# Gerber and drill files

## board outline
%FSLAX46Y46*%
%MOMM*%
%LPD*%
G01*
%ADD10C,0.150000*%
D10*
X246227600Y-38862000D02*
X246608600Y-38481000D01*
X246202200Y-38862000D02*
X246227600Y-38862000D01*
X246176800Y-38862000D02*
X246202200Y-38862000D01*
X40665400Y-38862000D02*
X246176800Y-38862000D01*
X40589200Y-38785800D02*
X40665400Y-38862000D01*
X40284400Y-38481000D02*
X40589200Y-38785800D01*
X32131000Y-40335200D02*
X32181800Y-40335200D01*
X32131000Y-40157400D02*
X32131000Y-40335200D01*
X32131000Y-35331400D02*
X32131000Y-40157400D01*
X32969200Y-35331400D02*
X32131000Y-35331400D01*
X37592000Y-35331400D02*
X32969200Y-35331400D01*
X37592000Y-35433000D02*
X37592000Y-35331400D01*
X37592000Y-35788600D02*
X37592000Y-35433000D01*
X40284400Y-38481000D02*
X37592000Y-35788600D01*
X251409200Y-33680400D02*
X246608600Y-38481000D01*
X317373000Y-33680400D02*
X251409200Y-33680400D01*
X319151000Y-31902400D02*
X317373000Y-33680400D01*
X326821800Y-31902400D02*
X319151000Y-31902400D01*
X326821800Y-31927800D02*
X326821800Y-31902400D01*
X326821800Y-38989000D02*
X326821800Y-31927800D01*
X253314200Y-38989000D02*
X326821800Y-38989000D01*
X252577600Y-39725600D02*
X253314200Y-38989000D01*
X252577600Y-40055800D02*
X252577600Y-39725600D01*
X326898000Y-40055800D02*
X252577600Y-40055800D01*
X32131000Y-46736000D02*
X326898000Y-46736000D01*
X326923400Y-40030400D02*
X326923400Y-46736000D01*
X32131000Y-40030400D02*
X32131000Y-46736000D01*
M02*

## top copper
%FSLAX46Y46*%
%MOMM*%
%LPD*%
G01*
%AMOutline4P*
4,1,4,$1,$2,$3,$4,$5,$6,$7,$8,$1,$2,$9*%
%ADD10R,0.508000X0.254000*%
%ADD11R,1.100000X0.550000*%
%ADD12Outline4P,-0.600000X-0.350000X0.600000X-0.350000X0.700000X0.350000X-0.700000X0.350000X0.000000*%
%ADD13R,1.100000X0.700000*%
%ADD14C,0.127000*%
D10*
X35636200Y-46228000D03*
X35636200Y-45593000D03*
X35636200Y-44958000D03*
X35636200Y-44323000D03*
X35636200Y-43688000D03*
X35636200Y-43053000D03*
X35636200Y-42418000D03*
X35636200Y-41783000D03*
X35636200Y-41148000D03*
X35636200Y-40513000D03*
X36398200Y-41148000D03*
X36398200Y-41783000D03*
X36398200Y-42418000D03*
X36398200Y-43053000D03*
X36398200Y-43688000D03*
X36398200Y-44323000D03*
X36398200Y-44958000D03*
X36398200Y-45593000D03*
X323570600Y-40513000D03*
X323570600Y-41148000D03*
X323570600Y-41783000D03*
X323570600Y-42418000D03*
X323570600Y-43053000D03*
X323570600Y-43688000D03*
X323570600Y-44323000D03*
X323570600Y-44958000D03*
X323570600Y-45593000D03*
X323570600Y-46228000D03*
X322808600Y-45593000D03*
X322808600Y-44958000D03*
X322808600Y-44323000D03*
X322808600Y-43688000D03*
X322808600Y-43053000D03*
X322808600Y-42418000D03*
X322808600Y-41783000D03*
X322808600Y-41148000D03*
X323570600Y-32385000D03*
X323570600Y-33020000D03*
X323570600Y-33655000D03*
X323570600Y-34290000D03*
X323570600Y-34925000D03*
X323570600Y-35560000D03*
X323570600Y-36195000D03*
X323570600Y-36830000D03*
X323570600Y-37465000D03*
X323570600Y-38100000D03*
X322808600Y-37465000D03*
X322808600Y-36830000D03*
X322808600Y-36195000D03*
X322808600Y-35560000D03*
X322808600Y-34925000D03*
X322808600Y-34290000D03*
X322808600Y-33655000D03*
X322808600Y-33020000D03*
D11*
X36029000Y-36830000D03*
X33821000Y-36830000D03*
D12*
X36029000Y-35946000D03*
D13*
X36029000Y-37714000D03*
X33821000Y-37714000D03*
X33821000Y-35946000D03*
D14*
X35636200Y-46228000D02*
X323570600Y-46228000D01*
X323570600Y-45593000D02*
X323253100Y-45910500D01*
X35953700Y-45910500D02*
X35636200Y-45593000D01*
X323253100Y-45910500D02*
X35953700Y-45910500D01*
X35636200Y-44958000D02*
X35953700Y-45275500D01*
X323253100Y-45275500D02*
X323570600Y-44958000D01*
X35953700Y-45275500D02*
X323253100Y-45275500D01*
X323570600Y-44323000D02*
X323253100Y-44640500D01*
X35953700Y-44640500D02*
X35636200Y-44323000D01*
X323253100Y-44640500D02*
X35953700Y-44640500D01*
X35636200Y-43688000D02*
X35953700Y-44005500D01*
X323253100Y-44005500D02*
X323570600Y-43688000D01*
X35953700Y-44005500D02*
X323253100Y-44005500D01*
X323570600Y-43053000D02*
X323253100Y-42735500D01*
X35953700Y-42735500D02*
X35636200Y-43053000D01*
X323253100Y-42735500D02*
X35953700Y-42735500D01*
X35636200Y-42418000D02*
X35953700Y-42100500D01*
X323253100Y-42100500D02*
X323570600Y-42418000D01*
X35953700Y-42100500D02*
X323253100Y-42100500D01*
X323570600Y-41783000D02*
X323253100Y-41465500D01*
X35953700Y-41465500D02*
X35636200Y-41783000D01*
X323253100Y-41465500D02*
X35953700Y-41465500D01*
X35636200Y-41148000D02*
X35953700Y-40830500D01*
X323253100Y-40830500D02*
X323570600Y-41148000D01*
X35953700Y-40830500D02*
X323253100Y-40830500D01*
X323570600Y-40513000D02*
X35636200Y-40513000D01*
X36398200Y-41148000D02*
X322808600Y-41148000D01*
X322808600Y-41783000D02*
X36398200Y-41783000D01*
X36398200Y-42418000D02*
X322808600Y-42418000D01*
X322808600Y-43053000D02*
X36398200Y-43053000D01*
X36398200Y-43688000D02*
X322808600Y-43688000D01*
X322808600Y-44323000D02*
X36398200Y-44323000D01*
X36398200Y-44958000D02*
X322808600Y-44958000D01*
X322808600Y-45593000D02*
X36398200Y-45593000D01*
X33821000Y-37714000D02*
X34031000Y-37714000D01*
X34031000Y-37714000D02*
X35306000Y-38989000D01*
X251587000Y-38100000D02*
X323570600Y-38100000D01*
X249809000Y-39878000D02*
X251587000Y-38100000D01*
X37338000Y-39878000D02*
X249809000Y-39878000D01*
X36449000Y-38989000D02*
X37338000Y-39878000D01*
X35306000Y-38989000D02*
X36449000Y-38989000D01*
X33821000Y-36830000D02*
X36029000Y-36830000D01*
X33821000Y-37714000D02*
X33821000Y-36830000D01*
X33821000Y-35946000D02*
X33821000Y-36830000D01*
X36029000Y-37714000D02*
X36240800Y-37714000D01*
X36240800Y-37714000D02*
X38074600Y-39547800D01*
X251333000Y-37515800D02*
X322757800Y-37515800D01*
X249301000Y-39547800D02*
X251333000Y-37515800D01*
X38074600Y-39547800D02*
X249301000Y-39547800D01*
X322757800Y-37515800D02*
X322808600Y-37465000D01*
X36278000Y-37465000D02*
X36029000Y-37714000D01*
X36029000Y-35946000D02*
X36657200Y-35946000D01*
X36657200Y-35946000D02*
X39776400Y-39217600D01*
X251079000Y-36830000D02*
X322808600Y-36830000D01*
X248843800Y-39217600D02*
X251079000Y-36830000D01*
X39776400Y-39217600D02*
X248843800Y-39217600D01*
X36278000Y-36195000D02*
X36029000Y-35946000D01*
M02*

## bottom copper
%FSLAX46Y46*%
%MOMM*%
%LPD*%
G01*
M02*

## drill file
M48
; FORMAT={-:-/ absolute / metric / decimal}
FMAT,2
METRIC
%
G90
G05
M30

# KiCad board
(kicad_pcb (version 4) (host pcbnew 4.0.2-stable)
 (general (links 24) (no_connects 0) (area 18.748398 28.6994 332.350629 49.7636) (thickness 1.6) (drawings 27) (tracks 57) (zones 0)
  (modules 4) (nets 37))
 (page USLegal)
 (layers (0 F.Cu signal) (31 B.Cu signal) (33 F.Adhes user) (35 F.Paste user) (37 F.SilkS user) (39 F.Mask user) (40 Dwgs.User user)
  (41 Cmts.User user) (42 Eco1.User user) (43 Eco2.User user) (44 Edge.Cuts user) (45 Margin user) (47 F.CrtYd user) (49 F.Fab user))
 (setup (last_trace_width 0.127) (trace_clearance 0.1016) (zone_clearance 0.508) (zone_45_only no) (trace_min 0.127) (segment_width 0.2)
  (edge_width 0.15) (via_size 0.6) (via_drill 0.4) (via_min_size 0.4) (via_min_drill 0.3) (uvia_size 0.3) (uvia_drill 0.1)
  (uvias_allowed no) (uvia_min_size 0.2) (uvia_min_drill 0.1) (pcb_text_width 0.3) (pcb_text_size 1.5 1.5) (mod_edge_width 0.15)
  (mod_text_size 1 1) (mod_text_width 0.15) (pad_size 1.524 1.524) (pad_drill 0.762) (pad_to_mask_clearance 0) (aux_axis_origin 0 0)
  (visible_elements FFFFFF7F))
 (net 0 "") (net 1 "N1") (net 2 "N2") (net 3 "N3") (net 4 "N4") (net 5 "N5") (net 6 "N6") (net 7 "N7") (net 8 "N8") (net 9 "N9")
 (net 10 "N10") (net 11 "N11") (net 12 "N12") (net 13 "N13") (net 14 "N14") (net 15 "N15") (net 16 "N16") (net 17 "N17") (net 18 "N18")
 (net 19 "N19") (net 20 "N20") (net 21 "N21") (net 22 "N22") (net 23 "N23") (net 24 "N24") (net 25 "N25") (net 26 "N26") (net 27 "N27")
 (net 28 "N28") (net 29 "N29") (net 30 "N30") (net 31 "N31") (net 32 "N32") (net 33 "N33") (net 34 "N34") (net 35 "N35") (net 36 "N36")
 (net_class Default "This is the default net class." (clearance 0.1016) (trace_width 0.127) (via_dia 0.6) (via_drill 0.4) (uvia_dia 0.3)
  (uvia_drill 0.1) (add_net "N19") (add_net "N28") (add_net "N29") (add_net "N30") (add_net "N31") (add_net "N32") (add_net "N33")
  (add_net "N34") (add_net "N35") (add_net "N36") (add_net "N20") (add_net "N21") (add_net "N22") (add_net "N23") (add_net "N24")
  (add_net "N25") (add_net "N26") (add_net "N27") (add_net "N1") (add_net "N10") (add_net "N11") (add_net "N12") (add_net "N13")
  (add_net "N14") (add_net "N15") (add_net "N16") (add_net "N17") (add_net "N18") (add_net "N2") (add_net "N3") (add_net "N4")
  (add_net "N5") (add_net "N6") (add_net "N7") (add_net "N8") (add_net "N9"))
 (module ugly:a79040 (layer F.Cu) (at 33.4772 43.307)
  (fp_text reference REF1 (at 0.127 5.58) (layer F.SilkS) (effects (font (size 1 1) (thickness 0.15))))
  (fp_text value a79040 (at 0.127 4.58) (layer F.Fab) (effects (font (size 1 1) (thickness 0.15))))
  (pad 1 smd rect (at 2.159 2.921) (size 0.508 0.254) (layers F.Cu F.Paste F.Mask) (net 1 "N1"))
  (pad 2 smd rect (at 2.159 2.286) (size 0.508 0.254) (layers F.Cu F.Paste F.Mask) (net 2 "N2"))
  (pad 3 smd rect (at 2.159 1.651) (size 0.508 0.254) (layers F.Cu F.Paste F.Mask) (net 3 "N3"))
  (pad 4 smd rect (at 2.159 1.016) (size 0.508 0.254) (layers F.Cu F.Paste F.Mask) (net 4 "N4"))
  (pad 5 smd rect (at 2.159 0.381) (size 0.508 0.254) (layers F.Cu F.Paste F.Mask) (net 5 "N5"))
  (pad 6 smd rect (at 2.159 -0.254) (size 0.508 0.254) (layers F.Cu F.Paste F.Mask) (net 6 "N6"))
  (pad 7 smd rect (at 2.159 -0.889) (size 0.508 0.254) (layers F.Cu F.Paste F.Mask) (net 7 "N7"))
  (pad 8 smd rect (at 2.159 -1.524) (size 0.508 0.254) (layers F.Cu F.Paste F.Mask) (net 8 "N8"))
  (pad 9 smd rect (at 2.159 -2.159) (size 0.508 0.254) (layers F.Cu F.Paste F.Mask) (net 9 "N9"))
  (pad 10 smd rect (at 2.159 -2.794) (size 0.508 0.254) (layers F.Cu F.Paste F.Mask) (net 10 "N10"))
  (pad 11 smd rect (at 2.921 -2.159) (size 0.508 0.254) (layers F.Cu F.Paste F.Mask) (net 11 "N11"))
  (pad 12 smd rect (at 2.921 -1.524) (size 0.508 0.254) (layers F.Cu F.Paste F.Mask) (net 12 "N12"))
  (pad 13 smd rect (at 2.921 -0.889) (size 0.508 0.254) (layers F.Cu F.Paste F.Mask) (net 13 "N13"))
  (pad 14 smd rect (at 2.921 -0.254) (size 0.508 0.254) (layers F.Cu F.Paste F.Mask) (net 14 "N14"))
  (pad 15 smd rect (at 2.921 0.381) (size 0.508 0.254) (layers F.Cu F.Paste F.Mask) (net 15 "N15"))
  (pad 16 smd rect (at 2.921 1.016) (size 0.508 0.254) (layers F.Cu F.Paste F.Mask) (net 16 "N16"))
  (pad 17 smd rect (at 2.921 1.651) (size 0.508 0.254) (layers F.Cu F.Paste F.Mask) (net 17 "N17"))
  (pad 18 smd rect (at 2.921 2.286) (size 0.508 0.254) (layers F.Cu F.Paste F.Mask) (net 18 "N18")))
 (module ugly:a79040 (layer F.Cu) (at 325.7296 43.434 180)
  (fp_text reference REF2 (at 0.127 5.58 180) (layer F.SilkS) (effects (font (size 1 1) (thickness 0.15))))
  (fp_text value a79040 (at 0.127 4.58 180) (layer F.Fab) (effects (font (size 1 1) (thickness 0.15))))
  (pad 1 smd rect (at 2.159 2.921 180) (size 0.508 0.254) (layers F.Cu F.Paste F.Mask) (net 10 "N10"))
  (pad 2 smd rect (at 2.159 2.286 180) (size 0.508 0.254) (layers F.Cu F.Paste F.Mask) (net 9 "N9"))
  (pad 3 smd rect (at 2.159 1.651 180) (size 0.508 0.254) (layers F.Cu F.Paste F.Mask) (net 8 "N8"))
  (pad 4 smd rect (at 2.159 1.016 180) (size 0.508 0.254) (layers F.Cu F.Paste F.Mask) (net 7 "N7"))
  (pad 5 smd rect (at 2.159 0.381 180) (size 0.508 0.254) (layers F.Cu F.Paste F.Mask) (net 6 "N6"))
  (pad 6 smd rect (at 2.159 -0.254 180) (size 0.508 0.254) (layers F.Cu F.Paste F.Mask) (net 5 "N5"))
  (pad 7 smd rect (at 2.159 -0.889 180) (size 0.508 0.254) (layers F.Cu F.Paste F.Mask) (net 4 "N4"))
  (pad 8 smd rect (at 2.159 -1.524 180) (size 0.508 0.254) (layers F.Cu F.Paste F.Mask) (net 3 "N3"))
  (pad 9 smd rect (at 2.159 -2.159 180) (size 0.508 0.254) (layers F.Cu F.Paste F.Mask) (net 2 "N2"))
  (pad 10 smd rect (at 2.159 -2.794 180) (size 0.508 0.254) (layers F.Cu F.Paste F.Mask) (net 1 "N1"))
  (pad 11 smd rect (at 2.921 -2.159 180) (size 0.508 0.254) (layers F.Cu F.Paste F.Mask) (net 18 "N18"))
  (pad 12 smd rect (at 2.921 -1.524 180) (size 0.508 0.254) (layers F.Cu F.Paste F.Mask) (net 17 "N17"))
  (pad 13 smd rect (at 2.921 -0.889 180) (size 0.508 0.254) (layers F.Cu F.Paste F.Mask) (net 16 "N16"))
  (pad 14 smd rect (at 2.921 -0.254 180) (size 0.508 0.254) (layers F.Cu F.Paste F.Mask) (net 15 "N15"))
  (pad 15 smd rect (at 2.921 0.381 180) (size 0.508 0.254) (layers F.Cu F.Paste F.Mask) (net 14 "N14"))
  (pad 16 smd rect (at 2.921 1.016 180) (size 0.508 0.254) (layers F.Cu F.Paste F.Mask) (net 13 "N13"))
  (pad 17 smd rect (at 2.921 1.651 180) (size 0.508 0.254) (layers F.Cu F.Paste F.Mask) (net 12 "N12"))
  (pad 18 smd rect (at 2.921 2.286 180) (size 0.508 0.254) (layers F.Cu F.Paste F.Mask) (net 11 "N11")))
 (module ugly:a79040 (layer F.Cu) (at 325.7296 35.306 180)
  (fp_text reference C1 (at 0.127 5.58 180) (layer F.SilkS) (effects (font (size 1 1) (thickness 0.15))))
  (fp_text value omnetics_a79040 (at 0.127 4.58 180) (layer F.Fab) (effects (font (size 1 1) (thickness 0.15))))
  (pad 1 smd rect (at 2.159 2.921 180) (size 0.508 0.254) (layers F.Cu F.Paste F.Mask) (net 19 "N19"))
  (pad 2 smd rect (at 2.159 2.286 180) (size 0.508 0.254) (layers F.Cu F.Paste F.Mask) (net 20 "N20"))
  (pad 3 smd rect (at 2.159 1.651 180) (size 0.508 0.254) (layers F.Cu F.Paste F.Mask) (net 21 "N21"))
  (pad 4 smd rect (at 2.159 1.016 180) (size 0.508 0.254) (layers F.Cu F.Paste F.Mask) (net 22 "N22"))
  (pad 5 smd rect (at 2.159 0.381 180) (size 0.508 0.254) (layers F.Cu F.Paste F.Mask) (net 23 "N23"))
  (pad 6 smd rect (at 2.159 -0.254 180) (size 0.508 0.254) (layers F.Cu F.Paste F.Mask) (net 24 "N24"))
  (pad 7 smd rect (at 2.159 -0.889 180) (size 0.508 0.254) (layers F.Cu F.Paste F.Mask) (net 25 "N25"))
  (pad 8 smd rect (at 2.159 -1.524 180) (size 0.508 0.254) (layers F.Cu F.Paste F.Mask) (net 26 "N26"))
  (pad 9 smd rect (at 2.159 -2.159 180) (size 0.508 0.254) (layers F.Cu F.Paste F.Mask) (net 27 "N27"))
  (pad 10 smd rect (at 2.159 -2.794 180) (size 0.508 0.254) (layers F.Cu F.Paste F.Mask) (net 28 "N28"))
  (pad 11 smd rect (at 2.921 -2.159 180) (size 0.508 0.254) (layers F.Cu F.Paste F.Mask) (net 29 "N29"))
  (pad 12 smd rect (at 2.921 -1.524 180) (size 0.508 0.254) (layers F.Cu F.Paste F.Mask) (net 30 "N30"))
  (pad 13 smd rect (at 2.921 -0.889 180) (size 0.508 0.254) (layers F.Cu F.Paste F.Mask) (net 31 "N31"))
  (pad 14 smd rect (at 2.921 -0.254 180) (size 0.508 0.254) (layers F.Cu F.Paste F.Mask) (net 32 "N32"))
  (pad 15 smd rect (at 2.921 0.381 180) (size 0.508 0.254) (layers F.Cu F.Paste F.Mask) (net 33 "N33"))
  (pad 16 smd rect (at 2.921 1.016 180) (size 0.508 0.254) (layers F.Cu F.Paste F.Mask) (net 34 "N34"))
  (pad 17 smd rect (at 2.921 1.651 180) (size 0.508 0.254) (layers F.Cu F.Paste F.Mask) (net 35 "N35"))
  (pad 18 smd rect (at 2.921 2.286 180) (size 0.508 0.254) (layers F.Cu F.Paste F.Mask) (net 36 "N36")))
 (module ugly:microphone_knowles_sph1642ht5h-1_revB (layer F.Cu) (at 34.925 36.83)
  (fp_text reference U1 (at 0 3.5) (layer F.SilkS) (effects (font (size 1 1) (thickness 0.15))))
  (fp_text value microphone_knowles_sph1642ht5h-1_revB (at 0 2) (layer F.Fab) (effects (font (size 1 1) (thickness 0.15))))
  (pad 5 smd rect (at 1.104 0) (size 1.1 0.55) (layers F.Cu F.Paste F.Mask) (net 28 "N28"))
  (pad 2 smd rect (at -1.104 0) (size 1.1 0.55) (layers F.Cu F.Paste F.Mask) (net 28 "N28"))
  (pad 6 smd trapezoid (at 1.104 -0.884) (size 1.3 0.7) (rect_delta 0 -0.1) (layers F.Cu F.Paste F.Mask) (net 30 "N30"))
  (pad 4 smd rect (at 1.104 0.884) (size 1.1 0.7) (layers F.Cu F.Paste F.Mask) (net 29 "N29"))
  (pad 3 smd rect (at -1.104 0.884) (size 1.1 0.7) (layers F.Cu F.Paste F.Mask) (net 28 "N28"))
  (pad 1 smd rect (at -1.104 -0.884) (size 1.1 0.7) (layers F.Cu F.Paste F.Mask) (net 28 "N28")))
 (gr_line (start 246.2276 38.862) (end 246.6086 38.481) (angle 90) (layer Edge.Cuts) (width 0.15))
 (gr_line (start 246.2022 38.862) (end 246.2276 38.862) (angle 90) (layer Edge.Cuts) (width 0.15))
 (gr_line (start 246.1768 38.862) (end 246.2022 38.862) (angle 90) (layer Edge.Cuts) (width 0.15))
 (gr_line (start 40.6654 38.862) (end 246.1768 38.862) (angle 90) (layer Edge.Cuts) (width 0.15))
 (gr_line (start 40.5892 38.7858) (end 40.6654 38.862) (angle 90) (layer Edge.Cuts) (width 0.15))
 (gr_line (start 40.2844 38.481) (end 40.5892 38.7858) (angle 90) (layer Edge.Cuts) (width 0.15))
 (gr_line (start 32.131 40.3352) (end 32.1818 40.3352) (angle 90) (layer Edge.Cuts) (width 0.15))
 (gr_line (start 32.131 40.1574) (end 32.131 40.3352) (angle 90) (layer Edge.Cuts) (width 0.15))
 (gr_line (start 32.131 35.3314) (end 32.131 40.1574) (angle 90) (layer Edge.Cuts) (width 0.15))
 (gr_line (start 32.9692 35.3314) (end 32.131 35.3314) (angle 90) (layer Edge.Cuts) (width 0.15))
 (gr_line (start 37.592 35.3314) (end 32.9692 35.3314) (angle 90) (layer Edge.Cuts) (width 0.15))
 (gr_line (start 37.592 35.433) (end 37.592 35.3314) (angle 90) (layer Edge.Cuts) (width 0.15))
 (gr_line (start 37.592 35.7886) (end 37.592 35.433) (angle 90) (layer Edge.Cuts) (width 0.15))
 (gr_line (start 40.2844 38.481) (end 37.592 35.7886) (angle 90) (layer Edge.Cuts) (width 0.15))
 (gr_line (start 251.4092 33.6804) (end 246.6086 38.481) (angle 90) (layer Edge.Cuts) (width 0.15))
 (gr_line (start 317.373 33.6804) (end 251.4092 33.6804) (angle 90) (layer Edge.Cuts) (width 0.15))
 (gr_line (start 319.151 31.9024) (end 317.373 33.6804) (angle 90) (layer Edge.Cuts) (width 0.15))
 (gr_line (start 326.8218 31.9024) (end 319.151 31.9024) (angle 90) (layer Edge.Cuts) (width 0.15))
 (gr_line (start 326.8218 31.9278) (end 326.8218 31.9024) (angle 90) (layer Edge.Cuts) (width 0.15))
 (gr_line (start 326.8218 38.989) (end 326.8218 31.9278) (angle 90) (layer Edge.Cuts) (width 0.15))
 (gr_line (start 253.3142 38.989) (end 326.8218 38.989) (angle 90) (layer Edge.Cuts) (width 0.15))
 (gr_line (start 252.5776 39.7256) (end 253.3142 38.989) (angle 90) (layer Edge.Cuts) (width 0.15))
 (gr_line (start 252.5776 40.0558) (end 252.5776 39.7256) (angle 90) (layer Edge.Cuts) (width 0.15))
 (gr_line (start 326.898 40.0558) (end 252.5776 40.0558) (angle 90) (layer Edge.Cuts) (width 0.15))
 (gr_line (start 32.131 46.736) (end 326.898 46.736) (angle 90) (layer Edge.Cuts) (width 0.15))
 (gr_line (start 326.9234 40.0304) (end 326.9234 46.736) (angle 90) (layer Edge.Cuts) (width 0.15))
 (gr_line (start 32.131 40.0304) (end 32.131 46.736) (angle 90) (layer Edge.Cuts) (width 0.15))
 (segment (start 35.6362 46.228) (end 323.5706 46.228) (width 0.127) (layer F.Cu) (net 1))
 (segment (start 323.5706 45.593) (end 323.2531 45.9105) (width 0.127) (layer F.Cu) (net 2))
 (segment (start 35.9537 45.9105) (end 35.6362 45.593) (width 0.127) (layer F.Cu) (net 2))
 (segment (start 323.2531 45.9105) (end 35.9537 45.9105) (width 0.127) (layer F.Cu) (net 2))
 (segment (start 35.6362 44.958) (end 35.9537 45.2755) (width 0.127) (layer F.Cu) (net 3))
 (segment (start 323.2531 45.2755) (end 323.5706 44.958) (width 0.127) (layer F.Cu) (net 3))
 (segment (start 35.9537 45.2755) (end 323.2531 45.2755) (width 0.127) (layer F.Cu) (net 3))
 (segment (start 323.5706 44.323) (end 323.2531 44.6405) (width 0.127) (layer F.Cu) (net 4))
 (segment (start 35.9537 44.6405) (end 35.6362 44.323) (width 0.127) (layer F.Cu) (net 4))
 (segment (start 323.2531 44.6405) (end 35.9537 44.6405) (width 0.127) (layer F.Cu) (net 4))
 (segment (start 35.6362 43.688) (end 35.9537 44.0055) (width 0.127) (layer F.Cu) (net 5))
 (segment (start 323.2531 44.0055) (end 323.5706 43.688) (width 0.127) (layer F.Cu) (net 5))
 (segment (start 35.9537 44.0055) (end 323.2531 44.0055) (width 0.127) (layer F.Cu) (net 5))
 (segment (start 323.5706 43.053) (end 323.2531 42.7355) (width 0.127) (layer F.Cu) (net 6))
 (segment (start 35.9537 42.7355) (end 35.6362 43.053) (width 0.127) (layer F.Cu) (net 6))
 (segment (start 323.2531 42.7355) (end 35.9537 42.7355) (width 0.127) (layer F.Cu) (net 6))
 (segment (start 35.6362 42.418) (end 35.9537 42.1005) (width 0.127) (layer F.Cu) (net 7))
 (segment (start 323.2531 42.1005) (end 323.5706 42.418) (width 0.127) (layer F.Cu) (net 7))
 (segment (start 35.9537 42.1005) (end 323.2531 42.1005) (width 0.127) (layer F.Cu) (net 7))
 (segment (start 323.5706 41.783) (end 323.2531 41.4655) (width 0.127) (layer F.Cu) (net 8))
 (segment (start 35.9537 41.4655) (end 35.6362 41.783) (width 0.127) (layer F.Cu) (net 8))
 (segment (start 323.2531 41.4655) (end 35.9537 41.4655) (width 0.127) (layer F.Cu) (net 8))
 (segment (start 35.6362 41.148) (end 35.9537 40.8305) (width 0.127) (layer F.Cu) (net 9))
 (segment (start 323.2531 40.8305) (end 323.5706 41.148) (width 0.127) (layer F.Cu) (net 9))
 (segment (start 35.9537 40.8305) (end 323.2531 40.8305) (width 0.127) (layer F.Cu) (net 9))
 (segment (start 323.5706 40.513) (end 35.6362 40.513) (width 0.127) (layer F.Cu) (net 10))
 (segment (start 36.3982 41.148) (end 322.8086 41.148) (width 0.127) (layer F.Cu) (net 11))
 (segment (start 322.8086 41.783) (end 36.3982 41.783) (width 0.127) (layer F.Cu) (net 12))
 (segment (start 36.3982 42.418) (end 322.8086 42.418) (width 0.127) (layer F.Cu) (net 13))
 (segment (start 322.8086 43.053) (end 36.3982 43.053) (width 0.127) (layer F.Cu) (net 14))
 (segment (start 36.3982 43.688) (end 322.8086 43.688) (width 0.127) (layer F.Cu) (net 15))
 (segment (start 322.8086 44.323) (end 36.3982 44.323) (width 0.127) (layer F.Cu) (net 16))
 (segment (start 36.3982 44.958) (end 322.8086 44.958) (width 0.127) (layer F.Cu) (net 17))
 (segment (start 322.8086 45.593) (end 36.3982 45.593) (width 0.127) (layer F.Cu) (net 18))
 (segment (start 33.821 37.714) (end 34.031 37.714) (width 0.127) (layer F.Cu) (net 28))
 (segment (start 34.031 37.714) (end 35.306 38.989) (width 0.127) (layer F.Cu) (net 28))
 (segment (start 251.587 38.1) (end 323.5706 38.1) (width 0.127) (layer F.Cu) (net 28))
 (segment (start 249.809 39.878) (end 251.587 38.1) (width 0.127) (layer F.Cu) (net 28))
 (segment (start 37.338 39.878) (end 249.809 39.878) (width 0.127) (layer F.Cu) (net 28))
 (segment (start 36.449 38.989) (end 37.338 39.878) (width 0.127) (layer F.Cu) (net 28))
 (segment (start 35.306 38.989) (end 36.449 38.989) (width 0.127) (layer F.Cu) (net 28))
 (segment (start 33.821 36.83) (end 36.029 36.83) (width 0.127) (layer F.Cu) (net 28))
 (segment (start 33.821 37.714) (end 33.821 36.83) (width 0.127) (layer F.Cu) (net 28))
 (segment (start 33.821 35.946) (end 33.821 36.83) (width 0.127) (layer F.Cu) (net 28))
 (segment (start 36.029 37.714) (end 36.2408 37.714) (width 0.127) (layer F.Cu) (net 29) (status C00000))
 (segment (start 36.2408 37.714) (end 38.0746 39.5478) (width 0.127) (layer F.Cu) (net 29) (status 400000))
 (segment (start 251.333 37.5158) (end 322.7578 37.5158) (width 0.127) (layer F.Cu) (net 29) (status 800000))
 (segment (start 249.301 39.5478) (end 251.333 37.5158) (width 0.127) (layer F.Cu) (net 29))
 (segment (start 38.0746 39.5478) (end 249.301 39.5478) (width 0.127) (layer F.Cu) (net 29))
 (segment (start 322.7578 37.5158) (end 322.8086 37.465) (width 0.127) (layer F.Cu) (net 29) (status C00000))
 (segment (start 36.278 37.465) (end 36.029 37.714) (width 0.127) (layer F.Cu) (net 29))
 (segment (start 36.029 35.946) (end 36.6572 35.946) (width 0.127) (layer F.Cu) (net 30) (status C00000))
 (segment (start 36.6572 35.946) (end 39.7764 39.2176) (width 0.127) (layer F.Cu) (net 30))
 (segment (start 251.079 36.83) (end 322.8086 36.83) (width 0.127) (layer F.Cu) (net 30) (status 800000))
 (segment (start 248.8438 39.2176) (end 251.079 36.83) (width 0.127) (layer F.Cu) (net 30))
 (segment (start 39.7764 39.2176) (end 248.8438 39.2176) (width 0.127) (layer F.Cu) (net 30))
 (segment (start 36.278 36.195) (end 36.029 35.946) (width 0.127) (layer F.Cu) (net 30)))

